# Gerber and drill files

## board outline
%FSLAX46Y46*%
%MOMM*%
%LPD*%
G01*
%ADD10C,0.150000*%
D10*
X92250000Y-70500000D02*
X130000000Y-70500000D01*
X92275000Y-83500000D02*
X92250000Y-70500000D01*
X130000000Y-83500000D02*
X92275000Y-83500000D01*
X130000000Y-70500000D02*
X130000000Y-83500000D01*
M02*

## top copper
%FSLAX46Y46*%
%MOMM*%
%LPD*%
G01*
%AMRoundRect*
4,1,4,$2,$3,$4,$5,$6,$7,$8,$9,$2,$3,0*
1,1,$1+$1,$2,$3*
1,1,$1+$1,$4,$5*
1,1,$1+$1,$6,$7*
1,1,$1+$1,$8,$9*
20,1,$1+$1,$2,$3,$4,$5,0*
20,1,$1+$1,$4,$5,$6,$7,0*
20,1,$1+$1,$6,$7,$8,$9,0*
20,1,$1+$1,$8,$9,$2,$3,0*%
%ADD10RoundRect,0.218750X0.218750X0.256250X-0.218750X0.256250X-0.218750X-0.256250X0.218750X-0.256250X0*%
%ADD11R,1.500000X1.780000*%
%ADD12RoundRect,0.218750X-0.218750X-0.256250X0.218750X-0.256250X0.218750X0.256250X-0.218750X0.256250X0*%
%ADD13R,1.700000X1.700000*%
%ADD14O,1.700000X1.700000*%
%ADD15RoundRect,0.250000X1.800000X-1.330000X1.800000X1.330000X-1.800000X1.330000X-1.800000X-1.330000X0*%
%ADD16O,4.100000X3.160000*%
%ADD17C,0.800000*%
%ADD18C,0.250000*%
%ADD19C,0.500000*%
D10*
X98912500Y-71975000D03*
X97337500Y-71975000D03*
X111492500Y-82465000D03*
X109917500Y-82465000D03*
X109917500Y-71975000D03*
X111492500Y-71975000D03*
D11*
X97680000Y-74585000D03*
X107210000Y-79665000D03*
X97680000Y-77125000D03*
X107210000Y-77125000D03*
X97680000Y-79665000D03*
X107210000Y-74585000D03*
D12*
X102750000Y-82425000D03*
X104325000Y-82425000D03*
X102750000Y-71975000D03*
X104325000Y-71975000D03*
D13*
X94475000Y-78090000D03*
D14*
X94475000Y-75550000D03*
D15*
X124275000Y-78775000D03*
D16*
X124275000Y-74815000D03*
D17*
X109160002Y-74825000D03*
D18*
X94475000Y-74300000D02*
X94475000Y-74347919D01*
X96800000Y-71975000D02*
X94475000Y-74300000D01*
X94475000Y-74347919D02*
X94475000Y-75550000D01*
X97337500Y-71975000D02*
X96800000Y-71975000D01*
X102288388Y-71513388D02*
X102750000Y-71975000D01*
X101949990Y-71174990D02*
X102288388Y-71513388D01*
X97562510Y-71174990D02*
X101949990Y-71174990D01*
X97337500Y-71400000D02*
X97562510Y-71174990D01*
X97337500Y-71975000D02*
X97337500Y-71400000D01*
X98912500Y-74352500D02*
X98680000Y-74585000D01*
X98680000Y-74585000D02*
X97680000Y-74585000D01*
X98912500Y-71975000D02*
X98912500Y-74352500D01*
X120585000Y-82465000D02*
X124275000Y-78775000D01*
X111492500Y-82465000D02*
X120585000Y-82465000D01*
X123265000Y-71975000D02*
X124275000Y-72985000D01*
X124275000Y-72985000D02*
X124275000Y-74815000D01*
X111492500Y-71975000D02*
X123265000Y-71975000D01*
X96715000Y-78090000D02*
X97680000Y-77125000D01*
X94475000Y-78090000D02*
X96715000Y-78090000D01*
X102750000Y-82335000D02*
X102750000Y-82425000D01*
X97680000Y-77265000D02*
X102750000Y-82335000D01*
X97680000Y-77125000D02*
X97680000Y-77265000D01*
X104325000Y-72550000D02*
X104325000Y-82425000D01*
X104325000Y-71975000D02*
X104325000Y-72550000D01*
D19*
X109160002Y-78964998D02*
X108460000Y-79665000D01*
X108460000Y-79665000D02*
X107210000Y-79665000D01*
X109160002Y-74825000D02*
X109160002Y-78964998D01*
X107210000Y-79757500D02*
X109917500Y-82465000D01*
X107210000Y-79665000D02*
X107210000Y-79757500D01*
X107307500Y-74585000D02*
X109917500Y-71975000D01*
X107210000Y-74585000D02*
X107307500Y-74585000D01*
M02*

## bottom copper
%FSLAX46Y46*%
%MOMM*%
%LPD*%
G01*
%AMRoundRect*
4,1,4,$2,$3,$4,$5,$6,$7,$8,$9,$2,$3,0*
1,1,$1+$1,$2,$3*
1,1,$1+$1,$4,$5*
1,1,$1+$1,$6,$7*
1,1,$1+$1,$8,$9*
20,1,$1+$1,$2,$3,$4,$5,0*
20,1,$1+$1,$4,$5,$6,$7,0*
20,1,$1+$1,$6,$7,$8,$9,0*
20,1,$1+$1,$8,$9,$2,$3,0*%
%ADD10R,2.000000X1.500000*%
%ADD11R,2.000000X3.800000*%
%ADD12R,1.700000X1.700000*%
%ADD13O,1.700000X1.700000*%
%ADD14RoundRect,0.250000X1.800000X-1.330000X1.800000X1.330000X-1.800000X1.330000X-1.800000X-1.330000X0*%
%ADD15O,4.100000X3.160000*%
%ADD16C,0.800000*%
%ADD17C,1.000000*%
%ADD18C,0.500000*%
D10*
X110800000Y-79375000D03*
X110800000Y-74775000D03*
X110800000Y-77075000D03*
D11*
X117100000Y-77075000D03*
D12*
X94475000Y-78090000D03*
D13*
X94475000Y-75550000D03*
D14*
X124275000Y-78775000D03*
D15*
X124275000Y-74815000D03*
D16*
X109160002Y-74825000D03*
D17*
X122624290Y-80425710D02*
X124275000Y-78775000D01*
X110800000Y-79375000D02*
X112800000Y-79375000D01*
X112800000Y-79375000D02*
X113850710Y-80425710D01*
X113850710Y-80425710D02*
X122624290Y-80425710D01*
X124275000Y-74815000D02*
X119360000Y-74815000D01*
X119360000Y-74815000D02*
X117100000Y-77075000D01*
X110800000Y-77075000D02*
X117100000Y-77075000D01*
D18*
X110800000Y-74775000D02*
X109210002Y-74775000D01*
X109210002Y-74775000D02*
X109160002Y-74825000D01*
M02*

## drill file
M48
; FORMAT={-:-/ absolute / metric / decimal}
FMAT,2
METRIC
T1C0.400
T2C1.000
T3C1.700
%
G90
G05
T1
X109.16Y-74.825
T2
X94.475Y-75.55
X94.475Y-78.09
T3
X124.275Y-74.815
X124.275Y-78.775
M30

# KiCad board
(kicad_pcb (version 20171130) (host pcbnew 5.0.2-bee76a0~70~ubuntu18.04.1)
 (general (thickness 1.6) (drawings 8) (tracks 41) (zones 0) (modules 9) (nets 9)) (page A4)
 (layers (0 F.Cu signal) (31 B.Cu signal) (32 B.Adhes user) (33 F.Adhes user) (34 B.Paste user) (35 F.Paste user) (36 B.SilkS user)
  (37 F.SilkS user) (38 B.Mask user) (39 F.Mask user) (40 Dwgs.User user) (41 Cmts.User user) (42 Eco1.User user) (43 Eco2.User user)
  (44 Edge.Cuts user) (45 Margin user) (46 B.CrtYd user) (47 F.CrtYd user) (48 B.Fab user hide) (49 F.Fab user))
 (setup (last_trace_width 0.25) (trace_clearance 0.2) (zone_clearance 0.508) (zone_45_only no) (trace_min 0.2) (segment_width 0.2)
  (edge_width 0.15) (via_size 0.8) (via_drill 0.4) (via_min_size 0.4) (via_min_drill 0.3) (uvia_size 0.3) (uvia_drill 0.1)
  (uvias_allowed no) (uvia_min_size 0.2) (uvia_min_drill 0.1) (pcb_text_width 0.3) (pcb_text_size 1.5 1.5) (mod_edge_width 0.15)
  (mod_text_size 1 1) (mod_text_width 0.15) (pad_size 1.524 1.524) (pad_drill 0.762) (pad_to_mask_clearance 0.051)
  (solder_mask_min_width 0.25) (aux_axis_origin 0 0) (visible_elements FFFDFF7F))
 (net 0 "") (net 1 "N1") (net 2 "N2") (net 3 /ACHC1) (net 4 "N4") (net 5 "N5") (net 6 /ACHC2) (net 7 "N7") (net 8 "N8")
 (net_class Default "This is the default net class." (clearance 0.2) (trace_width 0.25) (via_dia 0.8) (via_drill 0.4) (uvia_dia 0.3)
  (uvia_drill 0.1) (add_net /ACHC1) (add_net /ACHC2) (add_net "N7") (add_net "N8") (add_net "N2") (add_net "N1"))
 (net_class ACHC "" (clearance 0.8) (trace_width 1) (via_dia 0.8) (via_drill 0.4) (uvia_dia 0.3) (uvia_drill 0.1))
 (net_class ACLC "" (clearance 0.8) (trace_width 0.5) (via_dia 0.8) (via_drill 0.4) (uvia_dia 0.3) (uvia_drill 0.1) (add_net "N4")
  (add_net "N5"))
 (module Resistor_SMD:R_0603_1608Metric (layer F.Cu) (at 98.125 71.975 180)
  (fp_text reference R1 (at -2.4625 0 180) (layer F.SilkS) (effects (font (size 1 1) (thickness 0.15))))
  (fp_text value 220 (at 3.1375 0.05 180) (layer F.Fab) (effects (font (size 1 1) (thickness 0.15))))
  (pad 1 smd roundrect (at -0.7875 0 180) (size 0.875 0.95) (layers F.Cu F.Paste F.Mask) (roundrect_rratio 0.25) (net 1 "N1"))
  (pad 2 smd roundrect (at 0.7875 0 180) (size 0.875 0.95) (layers F.Cu F.Paste F.Mask) (roundrect_rratio 0.25) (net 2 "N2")))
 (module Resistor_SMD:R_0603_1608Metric (layer F.Cu) (at 110.705 82.465 180)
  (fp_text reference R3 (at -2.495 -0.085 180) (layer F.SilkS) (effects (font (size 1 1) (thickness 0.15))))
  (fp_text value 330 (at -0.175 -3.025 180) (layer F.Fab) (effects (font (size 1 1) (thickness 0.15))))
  (pad 1 smd roundrect (at -0.7875 0 180) (size 0.875 0.95) (layers F.Cu F.Paste F.Mask) (roundrect_rratio 0.25) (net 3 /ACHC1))
  (pad 2 smd roundrect (at 0.7875 0 180) (size 0.875 0.95) (layers F.Cu F.Paste F.Mask) (roundrect_rratio 0.25) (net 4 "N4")))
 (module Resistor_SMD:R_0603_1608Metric (layer F.Cu) (at 110.705 71.975 180)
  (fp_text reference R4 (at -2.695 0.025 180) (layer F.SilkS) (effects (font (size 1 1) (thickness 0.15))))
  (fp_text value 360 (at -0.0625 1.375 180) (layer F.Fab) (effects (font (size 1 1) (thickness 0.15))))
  (pad 2 smd roundrect (at 0.7875 0 180) (size 0.875 0.95) (layers F.Cu F.Paste F.Mask) (roundrect_rratio 0.25) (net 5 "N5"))
  (pad 1 smd roundrect (at -0.7875 0 180) (size 0.875 0.95) (layers F.Cu F.Paste F.Mask) (roundrect_rratio 0.25) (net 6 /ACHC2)))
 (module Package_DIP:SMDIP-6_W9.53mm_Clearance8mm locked (layer F.Cu) (at 102.445 77.125)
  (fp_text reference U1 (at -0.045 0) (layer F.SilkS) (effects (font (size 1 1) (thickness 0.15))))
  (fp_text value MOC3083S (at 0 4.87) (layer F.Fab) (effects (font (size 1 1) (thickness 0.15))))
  (pad 1 smd rect (at -4.765 -2.54) (size 1.5 1.78) (layers F.Cu F.Paste F.Mask) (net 1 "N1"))
  (pad 4 smd rect (at 4.765 2.54) (size 1.5 1.78) (layers F.Cu F.Paste F.Mask) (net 4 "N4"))
  (pad 2 smd rect (at -4.765 0) (size 1.5 1.78) (layers F.Cu F.Paste F.Mask) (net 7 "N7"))
  (pad 5 smd rect (at 4.765 0) (size 1.5 1.78) (layers F.Cu F.Paste F.Mask))
  (pad 3 smd rect (at -4.765 2.54) (size 1.5 1.78) (layers F.Cu F.Paste F.Mask))
  (pad 6 smd rect (at 4.765 -2.54) (size 1.5 1.78) (layers F.Cu F.Paste F.Mask) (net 5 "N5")))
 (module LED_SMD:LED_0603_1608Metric (layer F.Cu) (at 103.5375 82.425)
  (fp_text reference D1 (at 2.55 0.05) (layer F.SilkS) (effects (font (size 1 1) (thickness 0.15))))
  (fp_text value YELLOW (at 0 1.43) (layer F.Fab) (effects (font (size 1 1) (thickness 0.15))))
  (pad 1 smd roundrect (at -0.7875 0) (size 0.875 0.95) (layers F.Cu F.Paste F.Mask) (roundrect_rratio 0.25) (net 7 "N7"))
  (pad 2 smd roundrect (at 0.7875 0) (size 0.875 0.95) (layers F.Cu F.Paste F.Mask) (roundrect_rratio 0.25) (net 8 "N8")))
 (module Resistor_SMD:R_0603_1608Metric (layer F.Cu) (at 103.5375 71.975)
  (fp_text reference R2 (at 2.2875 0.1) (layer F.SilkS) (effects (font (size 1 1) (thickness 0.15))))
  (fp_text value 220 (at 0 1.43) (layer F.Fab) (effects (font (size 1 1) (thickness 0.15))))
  (pad 1 smd roundrect (at -0.7875 0) (size 0.875 0.95) (layers F.Cu F.Paste F.Mask) (roundrect_rratio 0.25) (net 2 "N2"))
  (pad 2 smd roundrect (at 0.7875 0) (size 0.875 0.95) (layers F.Cu F.Paste F.Mask) (roundrect_rratio 0.25) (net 8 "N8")))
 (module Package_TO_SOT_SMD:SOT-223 (layer B.Cu) (at 113.95 77.075)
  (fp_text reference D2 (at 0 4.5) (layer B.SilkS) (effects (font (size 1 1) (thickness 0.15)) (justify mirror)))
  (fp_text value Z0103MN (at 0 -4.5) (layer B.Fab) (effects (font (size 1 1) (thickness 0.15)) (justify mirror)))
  (pad 1 smd rect (at -3.15 2.3) (size 2 1.5) (layers B.Cu B.Paste B.Mask) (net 3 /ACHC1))
  (pad 3 smd rect (at -3.15 -2.3) (size 2 1.5) (layers B.Cu B.Paste B.Mask) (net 4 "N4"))
  (pad 2 smd rect (at -3.15 0) (size 2 1.5) (layers B.Cu B.Paste B.Mask) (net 6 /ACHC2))
  (pad 4 smd rect (at 3.15 0) (size 2 3.8) (layers B.Cu B.Paste B.Mask) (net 6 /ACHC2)))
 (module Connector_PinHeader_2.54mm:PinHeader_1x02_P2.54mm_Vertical (layer F.Cu) (at 94.475 78.09 180)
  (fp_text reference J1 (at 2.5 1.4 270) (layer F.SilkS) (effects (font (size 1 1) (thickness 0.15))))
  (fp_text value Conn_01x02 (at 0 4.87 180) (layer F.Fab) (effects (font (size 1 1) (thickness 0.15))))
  (pad 1 thru_hole rect (at 0 0 180) (size 1.7 1.7) (drill 1) (layers *.Cu *.Mask) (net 7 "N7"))
  (pad 2 thru_hole oval (at 0 2.54 180) (size 1.7 1.7) (drill 1) (layers *.Cu *.Mask) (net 2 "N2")))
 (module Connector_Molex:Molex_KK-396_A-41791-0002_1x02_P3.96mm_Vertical (layer F.Cu) (at 124.275 78.775 90)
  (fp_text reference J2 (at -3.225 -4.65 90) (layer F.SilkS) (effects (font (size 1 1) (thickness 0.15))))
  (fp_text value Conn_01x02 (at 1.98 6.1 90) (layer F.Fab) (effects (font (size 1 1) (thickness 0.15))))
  (pad 1 thru_hole roundrect (at 0 0 90) (size 3.16 4.1) (drill 1.7) (layers *.Cu *.Mask) (roundrect_rratio 0.079114) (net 3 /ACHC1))
  (pad 2 thru_hole oval (at 3.96 0 90) (size 3.16 4.1) (drill 1.7) (layers *.Cu *.Mask) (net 6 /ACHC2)))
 (gr_line (start 92.25 70.5) (end 130 70.5) (layer Edge.Cuts) (width 0.15))
 (gr_line (start 92.275 83.5) (end 92.25 70.5) (layer Edge.Cuts) (width 0.15))
 (gr_line (start 130 83.5) (end 92.275 83.5) (layer Edge.Cuts) (width 0.15))
 (gr_line (start 130 70.5) (end 130 83.5) (layer Edge.Cuts) (width 0.15))
 (segment (start 94.475 74.3) (end 94.475 74.347919) (width 0.25) (layer F.Cu) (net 2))
 (segment (start 96.8 71.975) (end 94.475 74.3) (width 0.25) (layer F.Cu) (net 2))
 (segment (start 94.475 74.347919) (end 94.475 75.55) (width 0.25) (layer F.Cu) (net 2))
 (segment (start 97.3375 71.975) (end 96.8 71.975) (width 0.25) (layer F.Cu) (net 2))
 (segment (start 102.288388 71.513388) (end 102.75 71.975) (width 0.25) (layer F.Cu) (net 2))
 (segment (start 101.94999 71.17499) (end 102.288388 71.513388) (width 0.25) (layer F.Cu) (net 2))
 (segment (start 97.56251 71.17499) (end 101.94999 71.17499) (width 0.25) (layer F.Cu) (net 2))
 (segment (start 97.3375 71.4) (end 97.56251 71.17499) (width 0.25) (layer F.Cu) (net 2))
 (segment (start 97.3375 71.975) (end 97.3375 71.4) (width 0.25) (layer F.Cu) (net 2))
 (segment (start 98.9125 74.3525) (end 98.68 74.585) (width 0.25) (layer F.Cu) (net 1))
 (segment (start 98.68 74.585) (end 97.68 74.585) (width 0.25) (layer F.Cu) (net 1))
 (segment (start 98.9125 71.975) (end 98.9125 74.3525) (width 0.25) (layer F.Cu) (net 1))
 (segment (start 122.62429 80.42571) (end 124.275 78.775) (width 1) (layer B.Cu) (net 3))
 (segment (start 110.8 79.375) (end 112.8 79.375) (width 1) (layer B.Cu) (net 3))
 (segment (start 112.8 79.375) (end 113.85071 80.42571) (width 1) (layer B.Cu) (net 3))
 (segment (start 113.85071 80.42571) (end 122.62429 80.42571) (width 1) (layer B.Cu) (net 3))
 (segment (start 120.585 82.465) (end 124.275 78.775) (width 0.25) (layer F.Cu) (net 3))
 (segment (start 111.4925 82.465) (end 120.585 82.465) (width 0.25) (layer F.Cu) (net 3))
 (segment (start 124.275 74.815) (end 119.36 74.815) (width 1) (layer B.Cu) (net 6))
 (segment (start 119.36 74.815) (end 117.1 77.075) (width 1) (layer B.Cu) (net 6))
 (segment (start 110.8 77.075) (end 117.1 77.075) (width 1) (layer B.Cu) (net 6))
 (segment (start 123.265 71.975) (end 124.275 72.985) (width 0.25) (layer F.Cu) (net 6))
 (segment (start 124.275 72.985) (end 124.275 74.815) (width 0.25) (layer F.Cu) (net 6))
 (segment (start 111.4925 71.975) (end 123.265 71.975) (width 0.25) (layer F.Cu) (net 6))
 (segment (start 96.715 78.09) (end 97.68 77.125) (width 0.25) (layer F.Cu) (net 7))
 (segment (start 94.475 78.09) (end 96.715 78.09) (width 0.25) (layer F.Cu) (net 7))
 (segment (start 102.75 82.335) (end 102.75 82.425) (width 0.25) (layer F.Cu) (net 7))
 (segment (start 97.68 77.265) (end 102.75 82.335) (width 0.25) (layer F.Cu) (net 7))
 (segment (start 97.68 77.125) (end 97.68 77.265) (width 0.25) (layer F.Cu) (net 7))
 (segment (start 104.325 72.55) (end 104.325 82.425) (width 0.25) (layer F.Cu) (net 8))
 (segment (start 104.325 71.975) (end 104.325 72.55) (width 0.25) (layer F.Cu) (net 8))
 (via (at 109.160002 74.825) (size 0.8) (drill 0.4) (layers F.Cu B.Cu) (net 4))
 (segment (start 110.8 74.775) (end 109.210002 74.775) (width 0.5) (layer B.Cu) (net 4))
 (segment (start 109.210002 74.775) (end 109.160002 74.825) (width 0.5) (layer B.Cu) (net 4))
 (segment (start 109.160002 78.964998) (end 108.46 79.665) (width 0.5) (layer F.Cu) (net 4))
 (segment (start 108.46 79.665) (end 107.21 79.665) (width 0.5) (layer F.Cu) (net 4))
 (segment (start 109.160002 74.825) (end 109.160002 78.964998) (width 0.5) (layer F.Cu) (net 4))
 (segment (start 107.21 79.7575) (end 109.9175 82.465) (width 0.5) (layer F.Cu) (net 4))
 (segment (start 107.21 79.665) (end 107.21 79.7575) (width 0.5) (layer F.Cu) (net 4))
 (segment (start 107.3075 74.585) (end 109.9175 71.975) (width 0.5) (layer F.Cu) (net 5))
 (segment (start 107.21 74.585) (end 107.3075 74.585) (width 0.5) (layer F.Cu) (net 5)))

